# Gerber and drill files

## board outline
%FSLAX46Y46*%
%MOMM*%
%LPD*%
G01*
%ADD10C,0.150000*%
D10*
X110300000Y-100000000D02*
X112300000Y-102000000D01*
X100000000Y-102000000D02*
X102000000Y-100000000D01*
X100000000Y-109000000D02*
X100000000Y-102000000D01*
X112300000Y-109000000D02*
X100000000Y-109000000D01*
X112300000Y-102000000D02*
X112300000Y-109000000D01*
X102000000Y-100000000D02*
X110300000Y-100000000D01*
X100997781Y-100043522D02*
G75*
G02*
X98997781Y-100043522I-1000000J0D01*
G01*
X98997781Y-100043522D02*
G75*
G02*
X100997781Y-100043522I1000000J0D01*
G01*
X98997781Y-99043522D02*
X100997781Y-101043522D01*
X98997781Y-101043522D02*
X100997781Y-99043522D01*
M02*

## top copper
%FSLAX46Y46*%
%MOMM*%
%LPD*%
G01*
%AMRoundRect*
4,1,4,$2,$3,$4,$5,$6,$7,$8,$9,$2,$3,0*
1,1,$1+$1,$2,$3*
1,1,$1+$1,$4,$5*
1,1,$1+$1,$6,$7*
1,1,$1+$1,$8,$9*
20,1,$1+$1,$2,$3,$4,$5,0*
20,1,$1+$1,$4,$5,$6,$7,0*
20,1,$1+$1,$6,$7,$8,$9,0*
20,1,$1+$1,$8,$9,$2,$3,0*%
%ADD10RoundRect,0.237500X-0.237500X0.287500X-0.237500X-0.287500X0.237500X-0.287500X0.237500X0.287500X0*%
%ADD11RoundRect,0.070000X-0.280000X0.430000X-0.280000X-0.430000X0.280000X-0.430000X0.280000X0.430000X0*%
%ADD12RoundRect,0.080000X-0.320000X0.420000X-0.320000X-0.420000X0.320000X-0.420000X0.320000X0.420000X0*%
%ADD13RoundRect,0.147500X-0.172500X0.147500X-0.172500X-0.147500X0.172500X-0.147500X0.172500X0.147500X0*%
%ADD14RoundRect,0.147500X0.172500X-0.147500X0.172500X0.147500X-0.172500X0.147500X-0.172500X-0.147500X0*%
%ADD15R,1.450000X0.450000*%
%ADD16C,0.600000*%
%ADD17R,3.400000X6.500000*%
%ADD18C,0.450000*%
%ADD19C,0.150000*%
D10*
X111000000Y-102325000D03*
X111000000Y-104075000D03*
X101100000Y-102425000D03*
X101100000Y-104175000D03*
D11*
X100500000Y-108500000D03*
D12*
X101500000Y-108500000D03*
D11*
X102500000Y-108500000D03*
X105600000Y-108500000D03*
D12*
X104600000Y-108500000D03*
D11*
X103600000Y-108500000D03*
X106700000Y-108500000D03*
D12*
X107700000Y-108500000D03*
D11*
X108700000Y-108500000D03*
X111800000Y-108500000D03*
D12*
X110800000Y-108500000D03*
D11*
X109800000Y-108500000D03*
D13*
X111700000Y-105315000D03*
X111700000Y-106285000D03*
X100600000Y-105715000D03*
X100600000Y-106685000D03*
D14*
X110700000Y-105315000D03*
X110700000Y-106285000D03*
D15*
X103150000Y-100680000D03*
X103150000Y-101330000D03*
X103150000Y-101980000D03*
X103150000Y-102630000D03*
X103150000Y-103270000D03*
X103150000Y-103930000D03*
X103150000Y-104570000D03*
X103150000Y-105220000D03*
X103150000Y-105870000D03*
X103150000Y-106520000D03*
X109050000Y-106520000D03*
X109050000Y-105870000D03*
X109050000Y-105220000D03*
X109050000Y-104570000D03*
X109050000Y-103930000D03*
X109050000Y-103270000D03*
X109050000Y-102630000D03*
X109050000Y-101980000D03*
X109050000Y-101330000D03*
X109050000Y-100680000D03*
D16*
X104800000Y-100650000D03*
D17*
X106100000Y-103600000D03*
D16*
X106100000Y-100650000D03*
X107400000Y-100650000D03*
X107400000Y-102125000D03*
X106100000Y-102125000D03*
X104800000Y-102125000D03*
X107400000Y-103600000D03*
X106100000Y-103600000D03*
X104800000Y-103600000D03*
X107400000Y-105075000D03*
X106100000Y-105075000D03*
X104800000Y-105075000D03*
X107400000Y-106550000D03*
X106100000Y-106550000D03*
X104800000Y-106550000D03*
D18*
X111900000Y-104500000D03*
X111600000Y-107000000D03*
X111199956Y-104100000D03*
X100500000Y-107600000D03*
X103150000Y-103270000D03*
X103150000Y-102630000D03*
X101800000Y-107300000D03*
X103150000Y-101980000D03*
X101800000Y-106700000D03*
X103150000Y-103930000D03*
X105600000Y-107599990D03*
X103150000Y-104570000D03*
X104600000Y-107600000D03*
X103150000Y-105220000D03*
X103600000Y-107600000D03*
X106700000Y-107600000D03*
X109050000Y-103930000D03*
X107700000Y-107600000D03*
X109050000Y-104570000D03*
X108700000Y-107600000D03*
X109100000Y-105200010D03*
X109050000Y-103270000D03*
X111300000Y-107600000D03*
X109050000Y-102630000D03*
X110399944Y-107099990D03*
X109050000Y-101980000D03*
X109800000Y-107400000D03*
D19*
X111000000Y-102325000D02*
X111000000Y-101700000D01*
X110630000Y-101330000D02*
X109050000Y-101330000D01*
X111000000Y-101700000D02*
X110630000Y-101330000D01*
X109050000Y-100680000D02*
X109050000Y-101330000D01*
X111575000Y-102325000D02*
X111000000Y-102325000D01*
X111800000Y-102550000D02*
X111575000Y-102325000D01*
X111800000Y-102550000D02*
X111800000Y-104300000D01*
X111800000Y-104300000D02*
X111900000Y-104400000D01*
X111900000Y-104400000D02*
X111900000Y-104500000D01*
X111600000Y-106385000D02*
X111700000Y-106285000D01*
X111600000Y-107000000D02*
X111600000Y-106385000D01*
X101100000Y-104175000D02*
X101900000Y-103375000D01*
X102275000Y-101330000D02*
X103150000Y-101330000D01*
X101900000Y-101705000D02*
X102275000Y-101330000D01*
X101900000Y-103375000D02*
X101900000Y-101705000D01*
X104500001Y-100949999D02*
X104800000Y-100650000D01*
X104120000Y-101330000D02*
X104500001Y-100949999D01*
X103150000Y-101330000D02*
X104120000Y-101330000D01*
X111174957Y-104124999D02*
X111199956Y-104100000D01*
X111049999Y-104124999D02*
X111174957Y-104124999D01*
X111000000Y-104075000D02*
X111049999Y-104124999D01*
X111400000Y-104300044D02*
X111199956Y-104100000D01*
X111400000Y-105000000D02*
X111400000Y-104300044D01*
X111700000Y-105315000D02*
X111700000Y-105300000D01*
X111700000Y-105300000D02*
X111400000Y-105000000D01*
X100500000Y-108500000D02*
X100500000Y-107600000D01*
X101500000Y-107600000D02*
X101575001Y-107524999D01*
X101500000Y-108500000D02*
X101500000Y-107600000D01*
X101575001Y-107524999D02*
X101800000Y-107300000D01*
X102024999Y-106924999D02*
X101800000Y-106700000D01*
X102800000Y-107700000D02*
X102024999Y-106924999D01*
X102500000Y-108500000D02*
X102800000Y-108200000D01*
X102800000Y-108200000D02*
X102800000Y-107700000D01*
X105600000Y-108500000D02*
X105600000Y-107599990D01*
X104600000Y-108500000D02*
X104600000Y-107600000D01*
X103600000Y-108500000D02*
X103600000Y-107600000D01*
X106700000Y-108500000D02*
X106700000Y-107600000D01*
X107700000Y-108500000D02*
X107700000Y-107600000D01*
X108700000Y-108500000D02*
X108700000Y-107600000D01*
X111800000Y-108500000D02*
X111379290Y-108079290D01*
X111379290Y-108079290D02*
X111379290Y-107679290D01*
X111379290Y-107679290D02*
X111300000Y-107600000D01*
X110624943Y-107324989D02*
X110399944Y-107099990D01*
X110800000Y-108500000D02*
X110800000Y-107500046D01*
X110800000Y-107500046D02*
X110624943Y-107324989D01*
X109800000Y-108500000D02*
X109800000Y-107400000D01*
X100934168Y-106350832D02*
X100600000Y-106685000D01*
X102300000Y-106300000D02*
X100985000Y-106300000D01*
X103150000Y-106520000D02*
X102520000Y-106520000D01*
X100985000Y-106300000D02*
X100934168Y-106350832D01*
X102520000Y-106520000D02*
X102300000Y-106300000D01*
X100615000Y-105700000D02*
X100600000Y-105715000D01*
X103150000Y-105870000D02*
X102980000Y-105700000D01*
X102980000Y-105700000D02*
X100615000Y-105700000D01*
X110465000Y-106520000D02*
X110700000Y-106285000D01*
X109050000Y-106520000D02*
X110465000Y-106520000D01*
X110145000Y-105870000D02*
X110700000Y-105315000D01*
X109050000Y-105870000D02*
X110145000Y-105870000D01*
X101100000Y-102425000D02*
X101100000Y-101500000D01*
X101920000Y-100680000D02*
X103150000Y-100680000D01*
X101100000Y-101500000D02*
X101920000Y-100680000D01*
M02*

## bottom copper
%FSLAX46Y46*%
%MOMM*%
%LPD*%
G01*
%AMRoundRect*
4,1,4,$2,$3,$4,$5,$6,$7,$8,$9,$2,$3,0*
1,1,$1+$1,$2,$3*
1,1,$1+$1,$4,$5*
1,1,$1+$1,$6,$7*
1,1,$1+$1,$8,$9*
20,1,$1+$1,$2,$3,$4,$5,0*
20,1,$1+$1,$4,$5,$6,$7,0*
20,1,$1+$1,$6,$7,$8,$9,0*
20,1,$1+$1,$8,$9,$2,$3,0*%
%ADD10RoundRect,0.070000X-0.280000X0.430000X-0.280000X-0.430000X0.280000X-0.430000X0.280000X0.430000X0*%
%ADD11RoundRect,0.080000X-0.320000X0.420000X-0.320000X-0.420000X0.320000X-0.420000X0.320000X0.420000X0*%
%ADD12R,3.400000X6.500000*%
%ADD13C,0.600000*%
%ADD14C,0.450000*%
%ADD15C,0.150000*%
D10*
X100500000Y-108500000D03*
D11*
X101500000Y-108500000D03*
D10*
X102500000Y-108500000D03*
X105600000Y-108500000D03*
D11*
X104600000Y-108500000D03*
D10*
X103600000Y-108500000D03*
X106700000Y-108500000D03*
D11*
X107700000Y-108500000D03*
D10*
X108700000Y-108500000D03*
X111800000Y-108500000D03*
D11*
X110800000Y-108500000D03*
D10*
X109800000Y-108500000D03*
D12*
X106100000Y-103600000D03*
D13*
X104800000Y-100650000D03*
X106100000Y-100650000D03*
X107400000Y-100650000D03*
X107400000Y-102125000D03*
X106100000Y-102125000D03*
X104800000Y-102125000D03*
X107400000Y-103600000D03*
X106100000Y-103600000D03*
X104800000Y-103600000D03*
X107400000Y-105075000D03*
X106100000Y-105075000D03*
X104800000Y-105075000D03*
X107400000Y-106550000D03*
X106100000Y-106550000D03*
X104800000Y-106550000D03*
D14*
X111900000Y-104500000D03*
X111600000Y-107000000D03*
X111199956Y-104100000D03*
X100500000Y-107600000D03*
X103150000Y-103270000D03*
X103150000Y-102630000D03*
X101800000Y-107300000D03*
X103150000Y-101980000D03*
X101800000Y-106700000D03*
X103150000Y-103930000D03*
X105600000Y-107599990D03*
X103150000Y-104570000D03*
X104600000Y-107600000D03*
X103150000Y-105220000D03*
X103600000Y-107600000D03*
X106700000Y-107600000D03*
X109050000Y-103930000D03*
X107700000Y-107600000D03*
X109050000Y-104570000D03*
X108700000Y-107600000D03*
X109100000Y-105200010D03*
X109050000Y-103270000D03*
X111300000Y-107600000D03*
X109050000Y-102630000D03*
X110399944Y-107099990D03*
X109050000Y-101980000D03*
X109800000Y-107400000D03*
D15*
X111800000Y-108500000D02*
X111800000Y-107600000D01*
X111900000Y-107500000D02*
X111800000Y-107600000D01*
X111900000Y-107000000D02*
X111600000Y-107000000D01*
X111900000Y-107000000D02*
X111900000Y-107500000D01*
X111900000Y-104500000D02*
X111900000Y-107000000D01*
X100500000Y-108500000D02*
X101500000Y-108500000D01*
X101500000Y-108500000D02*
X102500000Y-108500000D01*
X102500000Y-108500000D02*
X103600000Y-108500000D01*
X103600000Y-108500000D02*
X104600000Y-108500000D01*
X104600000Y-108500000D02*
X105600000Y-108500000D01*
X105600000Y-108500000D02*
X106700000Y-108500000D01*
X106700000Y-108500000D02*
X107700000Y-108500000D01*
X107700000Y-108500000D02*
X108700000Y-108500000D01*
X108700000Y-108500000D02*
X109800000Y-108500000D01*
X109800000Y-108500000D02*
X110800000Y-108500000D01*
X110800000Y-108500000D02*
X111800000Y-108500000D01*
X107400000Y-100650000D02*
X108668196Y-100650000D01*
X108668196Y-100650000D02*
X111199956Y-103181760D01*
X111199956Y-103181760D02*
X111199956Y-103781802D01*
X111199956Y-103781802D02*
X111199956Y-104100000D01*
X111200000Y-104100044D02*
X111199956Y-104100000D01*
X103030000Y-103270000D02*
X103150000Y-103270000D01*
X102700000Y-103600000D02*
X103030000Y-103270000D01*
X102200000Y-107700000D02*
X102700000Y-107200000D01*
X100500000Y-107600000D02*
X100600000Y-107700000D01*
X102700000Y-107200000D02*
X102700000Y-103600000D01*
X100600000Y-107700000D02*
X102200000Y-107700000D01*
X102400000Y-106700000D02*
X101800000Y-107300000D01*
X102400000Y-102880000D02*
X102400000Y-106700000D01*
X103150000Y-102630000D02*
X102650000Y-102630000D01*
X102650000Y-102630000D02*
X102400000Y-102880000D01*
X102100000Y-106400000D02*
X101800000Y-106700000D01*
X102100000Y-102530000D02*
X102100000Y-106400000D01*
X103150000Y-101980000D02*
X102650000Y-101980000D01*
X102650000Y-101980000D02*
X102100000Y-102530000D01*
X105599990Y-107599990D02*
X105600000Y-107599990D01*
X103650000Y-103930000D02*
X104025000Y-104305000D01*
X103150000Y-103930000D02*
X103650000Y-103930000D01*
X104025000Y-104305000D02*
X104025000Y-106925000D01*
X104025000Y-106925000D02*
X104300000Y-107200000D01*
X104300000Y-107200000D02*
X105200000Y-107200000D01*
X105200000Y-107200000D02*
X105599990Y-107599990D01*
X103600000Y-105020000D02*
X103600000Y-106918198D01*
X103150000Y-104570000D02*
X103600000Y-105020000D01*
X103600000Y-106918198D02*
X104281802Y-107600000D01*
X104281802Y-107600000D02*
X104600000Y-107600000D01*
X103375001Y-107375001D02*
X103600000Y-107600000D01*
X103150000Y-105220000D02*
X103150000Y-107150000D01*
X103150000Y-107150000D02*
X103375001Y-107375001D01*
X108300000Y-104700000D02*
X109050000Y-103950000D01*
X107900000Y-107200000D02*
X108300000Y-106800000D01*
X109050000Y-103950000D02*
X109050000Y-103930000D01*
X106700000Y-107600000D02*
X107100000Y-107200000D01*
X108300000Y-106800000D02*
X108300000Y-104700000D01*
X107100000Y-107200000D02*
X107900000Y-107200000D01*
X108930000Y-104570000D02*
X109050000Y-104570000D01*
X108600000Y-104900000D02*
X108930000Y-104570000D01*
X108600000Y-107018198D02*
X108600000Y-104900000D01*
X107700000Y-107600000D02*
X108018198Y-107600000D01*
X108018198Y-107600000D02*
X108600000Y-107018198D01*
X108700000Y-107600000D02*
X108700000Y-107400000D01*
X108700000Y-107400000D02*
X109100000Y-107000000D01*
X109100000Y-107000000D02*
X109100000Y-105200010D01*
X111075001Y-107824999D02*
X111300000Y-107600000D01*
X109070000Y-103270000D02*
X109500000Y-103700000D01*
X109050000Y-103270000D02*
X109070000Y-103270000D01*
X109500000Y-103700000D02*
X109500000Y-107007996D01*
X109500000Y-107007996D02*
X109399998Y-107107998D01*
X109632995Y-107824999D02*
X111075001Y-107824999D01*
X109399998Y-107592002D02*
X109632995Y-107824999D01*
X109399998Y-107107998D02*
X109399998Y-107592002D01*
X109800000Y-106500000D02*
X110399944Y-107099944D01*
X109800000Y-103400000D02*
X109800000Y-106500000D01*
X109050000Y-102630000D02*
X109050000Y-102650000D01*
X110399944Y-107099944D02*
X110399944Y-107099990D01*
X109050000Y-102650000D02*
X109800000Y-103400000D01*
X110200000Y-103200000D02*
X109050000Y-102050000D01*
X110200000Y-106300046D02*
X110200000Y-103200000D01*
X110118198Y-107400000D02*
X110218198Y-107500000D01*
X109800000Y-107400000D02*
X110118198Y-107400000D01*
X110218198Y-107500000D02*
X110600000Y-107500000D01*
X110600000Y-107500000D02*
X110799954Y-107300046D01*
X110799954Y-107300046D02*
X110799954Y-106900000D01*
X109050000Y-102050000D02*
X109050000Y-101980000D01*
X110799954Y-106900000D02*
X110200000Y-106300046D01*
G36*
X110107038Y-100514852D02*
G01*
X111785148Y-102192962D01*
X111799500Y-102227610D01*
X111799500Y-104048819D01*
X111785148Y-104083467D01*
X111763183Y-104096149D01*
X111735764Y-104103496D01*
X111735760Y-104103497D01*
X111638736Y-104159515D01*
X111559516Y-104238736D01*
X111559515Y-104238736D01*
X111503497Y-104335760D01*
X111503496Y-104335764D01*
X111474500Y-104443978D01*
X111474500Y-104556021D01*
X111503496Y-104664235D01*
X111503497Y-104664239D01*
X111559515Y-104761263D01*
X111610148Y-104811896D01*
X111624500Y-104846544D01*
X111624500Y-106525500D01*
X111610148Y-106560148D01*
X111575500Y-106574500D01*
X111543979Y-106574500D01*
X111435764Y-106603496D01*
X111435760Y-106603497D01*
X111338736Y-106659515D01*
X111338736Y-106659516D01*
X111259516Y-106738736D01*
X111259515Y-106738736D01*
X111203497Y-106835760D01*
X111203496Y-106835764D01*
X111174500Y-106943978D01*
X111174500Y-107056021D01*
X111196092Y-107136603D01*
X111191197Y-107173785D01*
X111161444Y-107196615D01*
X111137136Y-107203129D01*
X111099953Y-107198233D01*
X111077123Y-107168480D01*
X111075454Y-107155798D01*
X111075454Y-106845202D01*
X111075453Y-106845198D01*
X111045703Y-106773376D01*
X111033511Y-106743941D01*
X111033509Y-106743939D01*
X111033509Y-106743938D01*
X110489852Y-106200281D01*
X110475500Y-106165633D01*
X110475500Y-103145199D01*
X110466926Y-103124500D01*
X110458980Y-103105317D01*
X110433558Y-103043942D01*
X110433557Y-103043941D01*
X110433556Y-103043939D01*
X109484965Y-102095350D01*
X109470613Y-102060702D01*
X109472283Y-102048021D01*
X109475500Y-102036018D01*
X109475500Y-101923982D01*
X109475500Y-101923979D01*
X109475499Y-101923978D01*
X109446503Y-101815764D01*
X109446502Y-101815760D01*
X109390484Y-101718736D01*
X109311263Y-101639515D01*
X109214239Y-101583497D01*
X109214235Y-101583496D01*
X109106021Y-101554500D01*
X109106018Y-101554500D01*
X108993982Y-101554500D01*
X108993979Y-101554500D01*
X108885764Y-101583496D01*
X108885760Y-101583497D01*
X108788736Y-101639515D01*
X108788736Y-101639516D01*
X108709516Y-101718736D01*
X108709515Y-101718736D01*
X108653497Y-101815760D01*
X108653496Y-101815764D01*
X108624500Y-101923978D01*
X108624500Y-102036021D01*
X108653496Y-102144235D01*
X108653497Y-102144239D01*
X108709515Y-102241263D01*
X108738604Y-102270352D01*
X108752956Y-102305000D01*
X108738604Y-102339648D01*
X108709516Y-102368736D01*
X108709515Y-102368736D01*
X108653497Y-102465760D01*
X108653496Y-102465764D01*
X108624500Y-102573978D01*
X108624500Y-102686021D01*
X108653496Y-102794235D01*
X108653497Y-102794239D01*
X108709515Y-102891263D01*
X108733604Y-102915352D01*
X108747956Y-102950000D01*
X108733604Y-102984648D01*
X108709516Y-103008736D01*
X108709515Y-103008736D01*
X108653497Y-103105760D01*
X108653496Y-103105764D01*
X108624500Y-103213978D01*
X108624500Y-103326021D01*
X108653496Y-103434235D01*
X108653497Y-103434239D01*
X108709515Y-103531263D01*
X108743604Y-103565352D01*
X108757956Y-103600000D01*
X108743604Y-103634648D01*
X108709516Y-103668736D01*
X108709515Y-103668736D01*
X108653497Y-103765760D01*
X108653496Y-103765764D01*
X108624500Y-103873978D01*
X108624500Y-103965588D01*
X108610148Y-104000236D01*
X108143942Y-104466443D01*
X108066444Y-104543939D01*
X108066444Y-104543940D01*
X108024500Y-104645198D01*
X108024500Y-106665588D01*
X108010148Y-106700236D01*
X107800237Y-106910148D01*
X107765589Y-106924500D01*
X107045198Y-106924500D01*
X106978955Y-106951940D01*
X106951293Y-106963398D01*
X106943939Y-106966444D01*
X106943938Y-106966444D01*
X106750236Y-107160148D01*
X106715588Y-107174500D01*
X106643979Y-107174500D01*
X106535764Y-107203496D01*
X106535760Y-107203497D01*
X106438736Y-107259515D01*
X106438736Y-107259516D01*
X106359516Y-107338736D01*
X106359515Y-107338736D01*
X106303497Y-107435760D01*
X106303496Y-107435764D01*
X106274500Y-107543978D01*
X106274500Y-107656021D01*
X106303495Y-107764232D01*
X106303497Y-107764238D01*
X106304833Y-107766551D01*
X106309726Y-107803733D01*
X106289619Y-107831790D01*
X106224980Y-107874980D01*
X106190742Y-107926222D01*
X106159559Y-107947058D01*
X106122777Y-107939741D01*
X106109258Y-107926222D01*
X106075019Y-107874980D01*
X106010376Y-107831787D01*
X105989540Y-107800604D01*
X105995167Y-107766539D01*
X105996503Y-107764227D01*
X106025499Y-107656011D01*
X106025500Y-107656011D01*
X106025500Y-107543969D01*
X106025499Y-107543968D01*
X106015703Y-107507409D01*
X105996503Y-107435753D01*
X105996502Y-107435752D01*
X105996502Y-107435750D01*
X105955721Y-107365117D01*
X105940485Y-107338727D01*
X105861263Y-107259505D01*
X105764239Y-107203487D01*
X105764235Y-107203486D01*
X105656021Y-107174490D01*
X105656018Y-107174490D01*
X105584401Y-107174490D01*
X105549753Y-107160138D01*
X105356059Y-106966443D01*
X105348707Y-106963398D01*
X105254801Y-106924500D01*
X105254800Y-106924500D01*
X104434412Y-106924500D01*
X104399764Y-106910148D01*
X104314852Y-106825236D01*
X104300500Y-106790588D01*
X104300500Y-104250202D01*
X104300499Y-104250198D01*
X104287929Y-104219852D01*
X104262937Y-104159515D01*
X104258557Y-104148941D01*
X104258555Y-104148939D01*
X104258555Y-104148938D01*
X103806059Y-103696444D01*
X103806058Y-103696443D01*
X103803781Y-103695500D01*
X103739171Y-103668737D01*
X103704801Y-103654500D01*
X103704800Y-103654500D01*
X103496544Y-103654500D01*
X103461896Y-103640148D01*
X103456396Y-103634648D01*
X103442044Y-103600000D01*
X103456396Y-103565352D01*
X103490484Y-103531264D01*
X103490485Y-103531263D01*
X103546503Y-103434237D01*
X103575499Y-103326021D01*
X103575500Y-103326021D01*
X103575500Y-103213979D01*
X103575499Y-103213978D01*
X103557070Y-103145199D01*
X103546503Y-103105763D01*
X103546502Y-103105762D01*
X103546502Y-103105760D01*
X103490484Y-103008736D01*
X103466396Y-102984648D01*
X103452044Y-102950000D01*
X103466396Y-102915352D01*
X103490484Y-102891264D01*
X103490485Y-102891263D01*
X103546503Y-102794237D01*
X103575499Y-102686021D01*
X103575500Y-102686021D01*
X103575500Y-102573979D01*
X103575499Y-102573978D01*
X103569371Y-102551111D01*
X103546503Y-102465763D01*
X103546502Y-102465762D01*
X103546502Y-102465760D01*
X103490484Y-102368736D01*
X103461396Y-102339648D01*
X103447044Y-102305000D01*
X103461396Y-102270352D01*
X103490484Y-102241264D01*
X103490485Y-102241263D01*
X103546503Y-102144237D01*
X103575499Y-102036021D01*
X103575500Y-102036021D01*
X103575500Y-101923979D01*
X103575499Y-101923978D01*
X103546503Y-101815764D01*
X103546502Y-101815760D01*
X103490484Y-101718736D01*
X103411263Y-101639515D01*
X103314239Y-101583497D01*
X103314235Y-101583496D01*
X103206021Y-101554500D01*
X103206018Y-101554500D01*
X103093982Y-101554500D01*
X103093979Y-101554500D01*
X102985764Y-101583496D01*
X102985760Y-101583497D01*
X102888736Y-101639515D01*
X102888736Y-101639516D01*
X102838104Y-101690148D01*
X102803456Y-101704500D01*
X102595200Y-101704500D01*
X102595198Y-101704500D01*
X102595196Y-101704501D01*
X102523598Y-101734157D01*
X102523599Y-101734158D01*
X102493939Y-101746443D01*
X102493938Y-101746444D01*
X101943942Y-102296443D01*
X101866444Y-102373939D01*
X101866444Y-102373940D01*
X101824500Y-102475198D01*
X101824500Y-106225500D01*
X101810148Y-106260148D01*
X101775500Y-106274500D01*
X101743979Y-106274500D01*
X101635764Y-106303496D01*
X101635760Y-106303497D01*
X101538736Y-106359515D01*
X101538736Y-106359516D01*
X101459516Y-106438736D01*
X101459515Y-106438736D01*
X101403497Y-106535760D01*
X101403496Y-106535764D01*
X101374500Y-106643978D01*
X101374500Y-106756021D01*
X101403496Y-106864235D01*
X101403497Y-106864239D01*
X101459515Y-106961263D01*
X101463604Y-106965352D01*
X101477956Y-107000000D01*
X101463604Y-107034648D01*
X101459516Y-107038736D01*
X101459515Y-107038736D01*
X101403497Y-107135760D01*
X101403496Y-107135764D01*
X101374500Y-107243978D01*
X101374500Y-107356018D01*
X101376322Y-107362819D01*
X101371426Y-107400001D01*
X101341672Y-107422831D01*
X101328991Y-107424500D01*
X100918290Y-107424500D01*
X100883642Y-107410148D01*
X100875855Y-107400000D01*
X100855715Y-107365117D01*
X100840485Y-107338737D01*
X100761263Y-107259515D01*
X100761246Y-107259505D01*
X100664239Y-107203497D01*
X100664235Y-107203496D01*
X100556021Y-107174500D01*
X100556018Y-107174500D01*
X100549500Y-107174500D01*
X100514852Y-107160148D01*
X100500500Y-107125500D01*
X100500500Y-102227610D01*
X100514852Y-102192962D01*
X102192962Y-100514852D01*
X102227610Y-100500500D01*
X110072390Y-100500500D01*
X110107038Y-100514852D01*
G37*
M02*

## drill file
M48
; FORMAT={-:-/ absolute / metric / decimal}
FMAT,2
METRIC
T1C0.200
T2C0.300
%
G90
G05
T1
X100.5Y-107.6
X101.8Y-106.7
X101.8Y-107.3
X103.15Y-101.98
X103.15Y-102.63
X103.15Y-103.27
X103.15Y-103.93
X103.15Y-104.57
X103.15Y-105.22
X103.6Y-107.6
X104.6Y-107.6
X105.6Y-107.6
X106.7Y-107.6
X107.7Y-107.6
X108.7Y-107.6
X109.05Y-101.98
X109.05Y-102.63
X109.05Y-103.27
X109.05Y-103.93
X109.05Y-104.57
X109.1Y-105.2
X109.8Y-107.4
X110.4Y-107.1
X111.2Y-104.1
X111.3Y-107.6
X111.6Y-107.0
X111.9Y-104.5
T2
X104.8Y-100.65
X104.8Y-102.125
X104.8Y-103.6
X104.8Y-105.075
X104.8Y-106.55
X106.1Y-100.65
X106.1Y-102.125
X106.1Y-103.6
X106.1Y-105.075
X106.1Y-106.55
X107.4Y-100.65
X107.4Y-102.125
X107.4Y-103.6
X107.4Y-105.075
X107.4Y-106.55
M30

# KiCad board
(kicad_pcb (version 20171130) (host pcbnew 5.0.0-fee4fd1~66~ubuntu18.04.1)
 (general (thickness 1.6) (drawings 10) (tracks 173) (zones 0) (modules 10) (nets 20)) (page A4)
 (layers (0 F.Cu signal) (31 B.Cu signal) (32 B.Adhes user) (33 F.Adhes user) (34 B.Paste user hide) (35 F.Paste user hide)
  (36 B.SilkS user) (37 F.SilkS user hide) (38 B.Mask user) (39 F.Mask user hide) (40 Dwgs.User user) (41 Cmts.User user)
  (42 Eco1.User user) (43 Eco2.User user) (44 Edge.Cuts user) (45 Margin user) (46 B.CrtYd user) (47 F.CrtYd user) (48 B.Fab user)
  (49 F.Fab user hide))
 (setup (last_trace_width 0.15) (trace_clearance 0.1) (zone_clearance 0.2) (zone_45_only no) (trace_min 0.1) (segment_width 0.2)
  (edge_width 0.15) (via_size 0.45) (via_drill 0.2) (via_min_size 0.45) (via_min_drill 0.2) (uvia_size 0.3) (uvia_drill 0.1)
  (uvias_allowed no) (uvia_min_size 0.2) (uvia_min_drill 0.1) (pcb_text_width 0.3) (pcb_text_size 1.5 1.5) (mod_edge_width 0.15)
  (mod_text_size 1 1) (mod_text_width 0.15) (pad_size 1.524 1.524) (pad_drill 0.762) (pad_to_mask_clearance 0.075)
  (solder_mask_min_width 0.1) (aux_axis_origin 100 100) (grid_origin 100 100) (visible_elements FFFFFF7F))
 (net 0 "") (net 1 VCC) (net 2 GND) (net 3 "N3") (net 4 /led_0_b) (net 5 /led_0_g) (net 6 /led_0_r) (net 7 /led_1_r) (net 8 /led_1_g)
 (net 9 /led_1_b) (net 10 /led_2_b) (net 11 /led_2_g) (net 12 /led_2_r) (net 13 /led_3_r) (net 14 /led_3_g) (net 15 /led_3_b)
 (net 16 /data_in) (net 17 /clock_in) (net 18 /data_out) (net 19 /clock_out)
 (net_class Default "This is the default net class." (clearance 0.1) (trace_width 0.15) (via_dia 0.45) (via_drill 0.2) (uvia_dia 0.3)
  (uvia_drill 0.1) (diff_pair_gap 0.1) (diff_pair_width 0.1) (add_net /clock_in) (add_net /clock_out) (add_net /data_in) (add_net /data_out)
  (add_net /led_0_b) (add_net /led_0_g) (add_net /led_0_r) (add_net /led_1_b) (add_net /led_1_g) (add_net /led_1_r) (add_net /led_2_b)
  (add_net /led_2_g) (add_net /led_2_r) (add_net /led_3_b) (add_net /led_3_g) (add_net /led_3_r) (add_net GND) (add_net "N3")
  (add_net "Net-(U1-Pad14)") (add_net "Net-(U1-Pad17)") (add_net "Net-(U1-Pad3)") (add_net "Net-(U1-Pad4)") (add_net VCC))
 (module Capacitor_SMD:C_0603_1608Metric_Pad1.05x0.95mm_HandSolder (layer F.Cu) (at 111 103.2 270)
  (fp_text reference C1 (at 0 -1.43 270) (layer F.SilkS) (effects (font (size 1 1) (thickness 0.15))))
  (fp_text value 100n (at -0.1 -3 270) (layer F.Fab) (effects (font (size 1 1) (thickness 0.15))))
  (pad 1 smd roundrect (at -0.875 0 270) (size 1.05 0.95) (layers F.Cu F.Paste F.Mask) (roundrect_rratio 0.25) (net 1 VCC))
  (pad 2 smd roundrect (at 0.875 0 270) (size 1.05 0.95) (layers F.Cu F.Paste F.Mask) (roundrect_rratio 0.25) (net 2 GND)))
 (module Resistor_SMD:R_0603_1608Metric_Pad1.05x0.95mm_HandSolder (layer F.Cu) (at 101.1 103.3 270)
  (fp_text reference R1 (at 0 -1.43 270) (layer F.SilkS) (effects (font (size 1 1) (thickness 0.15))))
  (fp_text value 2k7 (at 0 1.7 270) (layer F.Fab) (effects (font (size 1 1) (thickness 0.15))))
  (pad 1 smd roundrect (at -0.875 0 270) (size 1.05 0.95) (layers F.Cu F.Paste F.Mask) (roundrect_rratio 0.25) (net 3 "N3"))
  (pad 2 smd roundrect (at 0.875 0 270) (size 1.05 0.95) (layers F.Cu F.Paste F.Mask) (roundrect_rratio 0.25) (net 2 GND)))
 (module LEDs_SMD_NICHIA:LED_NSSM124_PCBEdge (layer F.Cu) (at 101.5 109 270)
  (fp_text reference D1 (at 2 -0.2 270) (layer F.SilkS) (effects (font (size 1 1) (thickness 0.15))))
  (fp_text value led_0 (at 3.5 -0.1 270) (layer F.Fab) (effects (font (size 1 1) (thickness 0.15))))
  (pad 3 smd roundrect (at -0.5 1 270) (size 1 0.7) (layers F.Cu F.Mask) (roundrect_rratio 0.1) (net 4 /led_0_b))
  (pad 2 smd roundrect (at -0.5 0 270) (size 1 0.8) (layers F.Cu F.Mask) (roundrect_rratio 0.1) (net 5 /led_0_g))
  (pad 4 smd roundrect (at -0.5 1 270) (size 1 0.7) (layers B.Cu B.Mask) (roundrect_rratio 0.1) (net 1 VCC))
  (pad 5 smd roundrect (at -0.5 0 270) (size 1 0.8) (layers B.Cu B.Mask) (roundrect_rratio 0.1) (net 1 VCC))
  (pad 6 smd roundrect (at -0.5 -1 270) (size 1 0.7) (layers B.Cu B.Mask) (roundrect_rratio 0.1) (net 1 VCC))
  (pad 1 smd roundrect (at -0.5 -1 270) (size 1 0.7) (layers F.Cu F.Mask) (roundrect_rratio 0.1) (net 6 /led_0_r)))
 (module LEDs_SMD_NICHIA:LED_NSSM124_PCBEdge (layer F.Cu) (at 104.6 109 270)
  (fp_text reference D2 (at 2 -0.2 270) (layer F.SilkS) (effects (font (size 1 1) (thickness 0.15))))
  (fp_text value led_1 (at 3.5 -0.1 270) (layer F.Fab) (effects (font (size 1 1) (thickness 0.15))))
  (pad 1 smd roundrect (at -0.5 -1 270) (size 1 0.7) (layers F.Cu F.Mask) (roundrect_rratio 0.1) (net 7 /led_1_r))
  (pad 6 smd roundrect (at -0.5 -1 270) (size 1 0.7) (layers B.Cu B.Mask) (roundrect_rratio 0.1) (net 1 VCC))
  (pad 5 smd roundrect (at -0.5 0 270) (size 1 0.8) (layers B.Cu B.Mask) (roundrect_rratio 0.1) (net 1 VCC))
  (pad 4 smd roundrect (at -0.5 1 270) (size 1 0.7) (layers B.Cu B.Mask) (roundrect_rratio 0.1) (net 1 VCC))
  (pad 2 smd roundrect (at -0.5 0 270) (size 1 0.8) (layers F.Cu F.Mask) (roundrect_rratio 0.1) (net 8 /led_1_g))
  (pad 3 smd roundrect (at -0.5 1 270) (size 1 0.7) (layers F.Cu F.Mask) (roundrect_rratio 0.1) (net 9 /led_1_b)))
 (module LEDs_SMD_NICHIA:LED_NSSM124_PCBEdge (layer F.Cu) (at 107.7 109 270)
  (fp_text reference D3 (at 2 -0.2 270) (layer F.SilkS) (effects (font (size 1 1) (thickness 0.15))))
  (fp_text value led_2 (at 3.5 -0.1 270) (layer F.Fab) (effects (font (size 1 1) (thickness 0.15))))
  (pad 3 smd roundrect (at -0.5 1 270) (size 1 0.7) (layers F.Cu F.Mask) (roundrect_rratio 0.1) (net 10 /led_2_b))
  (pad 2 smd roundrect (at -0.5 0 270) (size 1 0.8) (layers F.Cu F.Mask) (roundrect_rratio 0.1) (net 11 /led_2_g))
  (pad 4 smd roundrect (at -0.5 1 270) (size 1 0.7) (layers B.Cu B.Mask) (roundrect_rratio 0.1) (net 1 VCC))
  (pad 5 smd roundrect (at -0.5 0 270) (size 1 0.8) (layers B.Cu B.Mask) (roundrect_rratio 0.1) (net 1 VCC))
  (pad 6 smd roundrect (at -0.5 -1 270) (size 1 0.7) (layers B.Cu B.Mask) (roundrect_rratio 0.1) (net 1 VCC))
  (pad 1 smd roundrect (at -0.5 -1 270) (size 1 0.7) (layers F.Cu F.Mask) (roundrect_rratio 0.1) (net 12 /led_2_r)))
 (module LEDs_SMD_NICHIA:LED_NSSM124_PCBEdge (layer F.Cu) (at 110.8 109 270)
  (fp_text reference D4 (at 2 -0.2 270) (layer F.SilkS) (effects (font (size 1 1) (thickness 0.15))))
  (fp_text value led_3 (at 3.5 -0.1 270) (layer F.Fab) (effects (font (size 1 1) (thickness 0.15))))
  (pad 1 smd roundrect (at -0.5 -1 270) (size 1 0.7) (layers F.Cu F.Mask) (roundrect_rratio 0.1) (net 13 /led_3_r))
  (pad 6 smd roundrect (at -0.5 -1 270) (size 1 0.7) (layers B.Cu B.Mask) (roundrect_rratio 0.1) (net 1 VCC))
  (pad 5 smd roundrect (at -0.5 0 270) (size 1 0.8) (layers B.Cu B.Mask) (roundrect_rratio 0.1) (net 1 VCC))
  (pad 4 smd roundrect (at -0.5 1 270) (size 1 0.7) (layers B.Cu B.Mask) (roundrect_rratio 0.1) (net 1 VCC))
  (pad 2 smd roundrect (at -0.5 0 270) (size 1 0.8) (layers F.Cu F.Mask) (roundrect_rratio 0.1) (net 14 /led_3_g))
  (pad 3 smd roundrect (at -0.5 1 270) (size 1 0.7) (layers F.Cu F.Mask) (roundrect_rratio 0.1) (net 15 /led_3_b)))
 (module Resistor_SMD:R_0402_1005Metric (layer F.Cu) (at 111.7 105.8 270)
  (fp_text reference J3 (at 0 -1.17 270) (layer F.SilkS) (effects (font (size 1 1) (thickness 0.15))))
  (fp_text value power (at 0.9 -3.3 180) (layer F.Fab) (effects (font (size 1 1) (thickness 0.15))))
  (pad 1 smd roundrect (at -0.485 0 270) (size 0.59 0.64) (layers F.Cu F.Paste F.Mask) (roundrect_rratio 0.25) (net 2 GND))
  (pad 2 smd roundrect (at 0.485 0 270) (size 0.59 0.64) (layers F.Cu F.Paste F.Mask) (roundrect_rratio 0.25) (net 1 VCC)))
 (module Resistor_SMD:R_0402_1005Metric (layer F.Cu) (at 100.6 106.2 270)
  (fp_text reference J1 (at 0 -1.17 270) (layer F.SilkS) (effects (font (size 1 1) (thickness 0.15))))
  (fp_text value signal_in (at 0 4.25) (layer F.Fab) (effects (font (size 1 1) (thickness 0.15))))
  (pad 1 smd roundrect (at -0.485 0 270) (size 0.59 0.64) (layers F.Cu F.Paste F.Mask) (roundrect_rratio 0.25) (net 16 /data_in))
  (pad 2 smd roundrect (at 0.485 0 270) (size 0.59 0.64) (layers F.Cu F.Paste F.Mask) (roundrect_rratio 0.25) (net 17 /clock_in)))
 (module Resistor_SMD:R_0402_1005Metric (layer F.Cu) (at 110.7 105.8 90)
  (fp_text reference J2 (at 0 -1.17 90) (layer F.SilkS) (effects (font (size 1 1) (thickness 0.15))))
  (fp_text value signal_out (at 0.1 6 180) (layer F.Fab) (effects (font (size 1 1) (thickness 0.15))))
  (pad 2 smd roundrect (at 0.485 0 90) (size 0.59 0.64) (layers F.Cu F.Paste F.Mask) (roundrect_rratio 0.25) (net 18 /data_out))
  (pad 1 smd roundrect (at -0.485 0 90) (size 0.59 0.64) (layers F.Cu F.Paste F.Mask) (roundrect_rratio 0.25) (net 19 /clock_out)))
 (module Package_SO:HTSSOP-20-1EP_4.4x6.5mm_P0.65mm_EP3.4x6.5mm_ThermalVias (layer F.Cu) (at 106.1 103.6)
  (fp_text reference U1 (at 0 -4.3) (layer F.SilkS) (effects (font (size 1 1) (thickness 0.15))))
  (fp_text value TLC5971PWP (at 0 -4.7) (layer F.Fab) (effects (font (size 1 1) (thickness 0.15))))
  (pad 21 smd rect (at 0 0) (size 3.4 6.5) (layers B.Cu) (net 2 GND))
  (pad 1 smd rect (at -2.95 -2.92) (size 1.45 0.45) (layers F.Cu F.Paste F.Mask) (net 3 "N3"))
  (pad 2 smd rect (at -2.95 -2.27) (size 1.45 0.45) (layers F.Cu F.Paste F.Mask) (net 2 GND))
  (pad 3 smd rect (at -2.95 -1.62) (size 1.45 0.45) (layers F.Cu F.Paste F.Mask) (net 6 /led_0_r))
  (pad 4 smd rect (at -2.95 -0.97) (size 1.45 0.45) (layers F.Cu F.Paste F.Mask) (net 5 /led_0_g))
  (pad 5 smd rect (at -2.95 -0.33) (size 1.45 0.45) (layers F.Cu F.Paste F.Mask) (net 4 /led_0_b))
  (pad 6 smd rect (at -2.95 0.33) (size 1.45 0.45) (layers F.Cu F.Paste F.Mask) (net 7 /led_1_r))
  (pad 7 smd rect (at -2.95 0.97) (size 1.45 0.45) (layers F.Cu F.Paste F.Mask) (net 8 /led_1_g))
  (pad 8 smd rect (at -2.95 1.62) (size 1.45 0.45) (layers F.Cu F.Paste F.Mask) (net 9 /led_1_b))
  (pad 9 smd rect (at -2.95 2.27) (size 1.45 0.45) (layers F.Cu F.Paste F.Mask) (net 16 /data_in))
  (pad 10 smd rect (at -2.95 2.92) (size 1.45 0.45) (layers F.Cu F.Paste F.Mask) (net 17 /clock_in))
  (pad 11 smd rect (at 2.95 2.92) (size 1.45 0.45) (layers F.Cu F.Paste F.Mask) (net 19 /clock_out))
  (pad 12 smd rect (at 2.95 2.27) (size 1.45 0.45) (layers F.Cu F.Paste F.Mask) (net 18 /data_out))
  (pad 13 smd rect (at 2.95 1.62) (size 1.45 0.45) (layers F.Cu F.Paste F.Mask) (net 12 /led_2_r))
  (pad 14 smd rect (at 2.95 0.97) (size 1.45 0.45) (layers F.Cu F.Paste F.Mask) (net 11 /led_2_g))
  (pad 15 smd rect (at 2.95 0.33) (size 1.45 0.45) (layers F.Cu F.Paste F.Mask) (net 10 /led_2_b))
  (pad 16 smd rect (at 2.95 -0.33) (size 1.45 0.45) (layers F.Cu F.Paste F.Mask) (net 13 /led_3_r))
  (pad 17 smd rect (at 2.95 -0.97) (size 1.45 0.45) (layers F.Cu F.Paste F.Mask) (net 14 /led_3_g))
  (pad 18 smd rect (at 2.95 -1.62) (size 1.45 0.45) (layers F.Cu F.Paste F.Mask) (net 15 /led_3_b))
  (pad 19 smd rect (at 2.95 -2.27) (size 1.45 0.45) (layers F.Cu F.Paste F.Mask) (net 1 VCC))
  (pad 20 smd rect (at 2.95 -2.92) (size 1.45 0.45) (layers F.Cu F.Paste F.Mask) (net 1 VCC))
  (pad 21 thru_hole circle (at -1.3 -2.95) (size 0.6 0.6) (drill 0.3) (layers *.Cu) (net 2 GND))
  (pad 21 smd rect (at 0 0) (size 3.4 6.5) (layers F.Cu F.Mask) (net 2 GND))
  (pad "" smd rect (at -0.85 -2.2125) (size 1.4 1.075) (layers F.Paste))
  (pad "" smd rect (at 0.85 -2.2125) (size 1.4 1.075) (layers F.Paste))
  (pad "" smd rect (at 0.85 -0.7375) (size 1.4 1.075) (layers F.Paste))
  (pad "" smd rect (at -0.85 -0.7375) (size 1.4 1.075) (layers F.Paste))
  (pad "" smd rect (at 0.85 0.7375) (size 1.4 1.075) (layers F.Paste))
  (pad "" smd rect (at -0.85 0.7375) (size 1.4 1.075) (layers F.Paste))
  (pad "" smd rect (at 0.85 2.2125) (size 1.4 1.075) (layers F.Paste))
  (pad "" smd rect (at -0.85 2.2125) (size 1.4 1.075) (layers F.Paste))
  (pad 21 thru_hole circle (at 0 -2.95) (size 0.6 0.6) (drill 0.3) (layers *.Cu) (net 2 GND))
  (pad 21 thru_hole circle (at 1.3 -2.95) (size 0.6 0.6) (drill 0.3) (layers *.Cu) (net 2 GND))
  (pad 21 thru_hole circle (at 1.3 -1.475) (size 0.6 0.6) (drill 0.3) (layers *.Cu) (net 2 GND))
  (pad 21 thru_hole circle (at 0 -1.475) (size 0.6 0.6) (drill 0.3) (layers *.Cu) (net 2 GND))
  (pad 21 thru_hole circle (at -1.3 -1.475) (size 0.6 0.6) (drill 0.3) (layers *.Cu) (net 2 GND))
  (pad 21 thru_hole circle (at 1.3 0) (size 0.6 0.6) (drill 0.3) (layers *.Cu) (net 2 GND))
  (pad 21 thru_hole circle (at 0 0) (size 0.6 0.6) (drill 0.3) (layers *.Cu) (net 2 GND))
  (pad 21 thru_hole circle (at -1.3 0) (size 0.6 0.6) (drill 0.3) (layers *.Cu) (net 2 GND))
  (pad 21 thru_hole circle (at 1.3 1.475) (size 0.6 0.6) (drill 0.3) (layers *.Cu) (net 2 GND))
  (pad 21 thru_hole circle (at 0 1.475) (size 0.6 0.6) (drill 0.3) (layers *.Cu) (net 2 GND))
  (pad 21 thru_hole circle (at -1.3 1.475) (size 0.6 0.6) (drill 0.3) (layers *.Cu) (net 2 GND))
  (pad 21 thru_hole circle (at 1.3 2.95) (size 0.6 0.6) (drill 0.3) (layers *.Cu) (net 2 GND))
  (pad 21 thru_hole circle (at 0 2.95) (size 0.6 0.6) (drill 0.3) (layers *.Cu) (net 2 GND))
  (pad 21 thru_hole circle (at -1.3 2.95) (size 0.6 0.6) (drill 0.3) (layers *.Cu) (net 2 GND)))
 (gr_line (start 110.3 100) (end 112.3 102) (layer Edge.Cuts) (width 0.15))
 (gr_line (start 100 102) (end 102 100) (layer Edge.Cuts) (width 0.15))
 (gr_line (start 100 109) (end 100 102) (layer Edge.Cuts) (width 0.15))
 (gr_line (start 112.3 109) (end 100 109) (layer Edge.Cuts) (width 0.15))
 (gr_line (start 112.3 102) (end 112.3 109) (layer Edge.Cuts) (width 0.15))
 (gr_line (start 102 100) (end 110.3 100) (layer Edge.Cuts) (width 0.15))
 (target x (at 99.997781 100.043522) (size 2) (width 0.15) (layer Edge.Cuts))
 (segment (start 111 102.325) (end 111 101.7) (width 0.15) (layer F.Cu) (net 1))
 (segment (start 110.63 101.33) (end 109.05 101.33) (width 0.15) (layer F.Cu) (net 1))
 (segment (start 111 101.7) (end 110.63 101.33) (width 0.15) (layer F.Cu) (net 1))
 (segment (start 109.05 100.68) (end 109.05 101.33) (width 0.15) (layer F.Cu) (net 1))
 (segment (start 111.575 102.325) (end 111 102.325) (width 0.15) (layer F.Cu) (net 1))
 (segment (start 111.8 102.55) (end 111.575 102.325) (width 0.15) (layer F.Cu) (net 1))
 (segment (start 111.8 108.5) (end 111.8 107.6) (width 0.15) (layer B.Cu) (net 1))
 (segment (start 111.8 102.55) (end 111.8 104.3) (width 0.15) (layer F.Cu) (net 1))
 (via (at 111.9 104.5) (size 0.45) (drill 0.2) (layers F.Cu B.Cu) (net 1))
 (segment (start 111.8 104.3) (end 111.9 104.4) (width 0.15) (layer F.Cu) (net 1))
 (segment (start 111.9 104.4) (end 111.9 104.5) (width 0.15) (layer F.Cu) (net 1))
 (segment (start 111.9 107.5) (end 111.8 107.6) (width 0.15) (layer B.Cu) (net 1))
 (segment (start 111.9 107) (end 111.6 107) (width 0.15) (layer B.Cu) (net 1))
 (segment (start 111.9 107) (end 111.9 107.5) (width 0.15) (layer B.Cu) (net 1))
 (via (at 111.6 107) (size 0.45) (drill 0.2) (layers F.Cu B.Cu) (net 1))
 (segment (start 111.9 104.5) (end 111.9 107) (width 0.15) (layer B.Cu) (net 1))
 (segment (start 111.6 106.385) (end 111.7 106.285) (width 0.15) (layer F.Cu) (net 1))
 (segment (start 111.6 107) (end 111.6 106.385) (width 0.15) (layer F.Cu) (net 1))
 (segment (start 100.5 108.5) (end 101.5 108.5) (width 0.15) (layer B.Cu) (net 1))
 (segment (start 101.5 108.5) (end 102.5 108.5) (width 0.15) (layer B.Cu) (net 1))
 (segment (start 102.5 108.5) (end 103.6 108.5) (width 0.15) (layer B.Cu) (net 1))
 (segment (start 103.6 108.5) (end 104.6 108.5) (width 0.15) (layer B.Cu) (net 1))
 (segment (start 104.6 108.5) (end 105.6 108.5) (width 0.15) (layer B.Cu) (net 1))
 (segment (start 105.6 108.5) (end 106.7 108.5) (width 0.15) (layer B.Cu) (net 1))
 (segment (start 106.7 108.5) (end 107.7 108.5) (width 0.15) (layer B.Cu) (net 1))
 (segment (start 107.7 108.5) (end 108.7 108.5) (width 0.15) (layer B.Cu) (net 1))
 (segment (start 108.7 108.5) (end 109.8 108.5) (width 0.15) (layer B.Cu) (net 1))
 (segment (start 109.8 108.5) (end 110.8 108.5) (width 0.15) (layer B.Cu) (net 1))
 (segment (start 110.8 108.5) (end 111.8 108.5) (width 0.15) (layer B.Cu) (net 1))
 (segment (start 101.1 104.175) (end 101.9 103.375) (width 0.15) (layer F.Cu) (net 2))
 (segment (start 102.275 101.33) (end 103.15 101.33) (width 0.15) (layer F.Cu) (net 2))
 (segment (start 101.9 101.705) (end 102.275 101.33) (width 0.15) (layer F.Cu) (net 2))
 (segment (start 101.9 103.375) (end 101.9 101.705) (width 0.15) (layer F.Cu) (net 2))
 (segment (start 104.500001 100.949999) (end 104.8 100.65) (width 0.15) (layer F.Cu) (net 2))
 (segment (start 104.12 101.33) (end 104.500001 100.949999) (width 0.15) (layer F.Cu) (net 2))
 (segment (start 103.15 101.33) (end 104.12 101.33) (width 0.15) (layer F.Cu) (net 2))
 (segment (start 107.4 100.65) (end 108.668196 100.65) (width 0.15) (layer B.Cu) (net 2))
 (segment (start 108.668196 100.65) (end 111.199956 103.18176) (width 0.15) (layer B.Cu) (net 2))
 (segment (start 111.174957 104.124999) (end 111.199956 104.1) (width 0.15) (layer F.Cu) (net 2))
 (via (at 111.199956 104.1) (size 0.45) (drill 0.2) (layers F.Cu B.Cu) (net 2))
 (segment (start 111.049999 104.124999) (end 111.174957 104.124999) (width 0.15) (layer F.Cu) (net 2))
 (segment (start 111.199956 103.18176) (end 111.199956 103.781802) (width 0.15) (layer B.Cu) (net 2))
 (segment (start 111 104.075) (end 111.049999 104.124999) (width 0.15) (layer F.Cu) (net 2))
 (segment (start 111.199956 103.781802) (end 111.199956 104.1) (width 0.15) (layer B.Cu) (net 2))
 (segment (start 111.2 104.100044) (end 111.199956 104.1) (width 0.15) (layer B.Cu) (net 2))
 (segment (start 111.4 104.300044) (end 111.199956 104.1) (width 0.15) (layer F.Cu) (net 2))
 (segment (start 111.4 105) (end 111.4 104.300044) (width 0.15) (layer F.Cu) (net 2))
 (segment (start 111.7 105.315) (end 111.7 105.3) (width 0.15) (layer F.Cu) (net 2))
 (segment (start 111.7 105.3) (end 111.4 105) (width 0.15) (layer F.Cu) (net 2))
 (via (at 100.5 107.6) (size 0.45) (drill 0.2) (layers F.Cu B.Cu) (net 4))
 (segment (start 100.5 108.5) (end 100.5 107.6) (width 0.15) (layer F.Cu) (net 4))
 (via (at 103.15 103.27) (size 0.45) (drill 0.2) (layers F.Cu B.Cu) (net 4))
 (segment (start 103.03 103.27) (end 103.15 103.27) (width 0.15) (layer B.Cu) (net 4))
 (segment (start 102.7 103.6) (end 103.03 103.27) (width 0.15) (layer B.Cu) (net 4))
 (segment (start 102.2 107.7) (end 102.7 107.2) (width 0.15) (layer B.Cu) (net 4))
 (segment (start 100.5 107.6) (end 100.6 107.7) (width 0.15) (layer B.Cu) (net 4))
 (segment (start 102.7 107.2) (end 102.7 103.6) (width 0.15) (layer B.Cu) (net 4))
 (segment (start 100.6 107.7) (end 102.2 107.7) (width 0.15) (layer B.Cu) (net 4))
 (via (at 103.15 102.63) (size 0.45) (drill 0.2) (layers F.Cu B.Cu) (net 5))
 (via (at 101.8 107.3) (size 0.45) (drill 0.2) (layers F.Cu B.Cu) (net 5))
 (segment (start 101.5 107.6) (end 101.575001 107.524999) (width 0.15) (layer F.Cu) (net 5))
 (segment (start 101.5 108.5) (end 101.5 107.6) (width 0.15) (layer F.Cu) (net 5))
 (segment (start 101.575001 107.524999) (end 101.8 107.3) (width 0.15) (layer F.Cu) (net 5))
 (segment (start 102.4 106.7) (end 101.8 107.3) (width 0.15) (layer B.Cu) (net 5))
 (segment (start 102.4 102.88) (end 102.4 106.7) (width 0.15) (layer B.Cu) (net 5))
 (segment (start 103.15 102.63) (end 102.65 102.63) (width 0.15) (layer B.Cu) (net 5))
 (segment (start 102.65 102.63) (end 102.4 102.88) (width 0.15) (layer B.Cu) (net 5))
 (via (at 103.15 101.98) (size 0.45) (drill 0.2) (layers F.Cu B.Cu) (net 6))
 (via (at 101.8 106.7) (size 0.45) (drill 0.2) (layers F.Cu B.Cu) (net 6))
 (segment (start 102.1 106.4) (end 101.8 106.7) (width 0.15) (layer B.Cu) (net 6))
 (segment (start 102.1 102.53) (end 102.1 106.4) (width 0.15) (layer B.Cu) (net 6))
 (segment (start 103.15 101.98) (end 102.65 101.98) (width 0.15) (layer B.Cu) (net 6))
 (segment (start 102.65 101.98) (end 102.1 102.53) (width 0.15) (layer B.Cu) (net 6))
 (segment (start 102.024999 106.924999) (end 101.8 106.7) (width 0.15) (layer F.Cu) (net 6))
 (segment (start 102.8 107.7) (end 102.024999 106.924999) (width 0.15) (layer F.Cu) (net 6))
 (segment (start 102.5 108.5) (end 102.8 108.2) (width 0.15) (layer F.Cu) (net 6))
 (segment (start 102.8 108.2) (end 102.8 107.7) (width 0.15) (layer F.Cu) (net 6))
 (via (at 103.15 103.93) (size 0.45) (drill 0.2) (layers F.Cu B.Cu) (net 7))
 (segment (start 105.6 108.5) (end 105.6 107.59999) (width 0.15) (layer F.Cu) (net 7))
 (via (at 105.6 107.59999) (size 0.45) (drill 0.2) (layers F.Cu B.Cu) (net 7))
 (segment (start 105.59999 107.59999) (end 105.6 107.59999) (width 0.15) (layer B.Cu) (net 7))
 (segment (start 103.65 103.93) (end 104.025 104.305) (width 0.15) (layer B.Cu) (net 7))
 (segment (start 103.15 103.93) (end 103.65 103.93) (width 0.15) (layer B.Cu) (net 7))
 (segment (start 104.025 104.305) (end 104.025 106.925) (width 0.15) (layer B.Cu) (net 7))
 (segment (start 104.025 106.925) (end 104.3 107.2) (width 0.15) (layer B.Cu) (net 7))
 (segment (start 104.3 107.2) (end 105.2 107.2) (width 0.15) (layer B.Cu) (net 7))
 (segment (start 105.2 107.2) (end 105.59999 107.59999) (width 0.15) (layer B.Cu) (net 7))
 (via (at 103.15 104.57) (size 0.45) (drill 0.2) (layers F.Cu B.Cu) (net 8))
 (segment (start 104.6 108.5) (end 104.6 107.6) (width 0.15) (layer F.Cu) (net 8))
 (via (at 104.6 107.6) (size 0.45) (drill 0.2) (layers F.Cu B.Cu) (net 8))
 (segment (start 103.6 105.02) (end 103.6 106.918198) (width 0.15) (layer B.Cu) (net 8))
 (segment (start 103.15 104.57) (end 103.6 105.02) (width 0.15) (layer B.Cu) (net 8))
 (segment (start 103.6 106.918198) (end 104.281802 107.6) (width 0.15) (layer B.Cu) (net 8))
 (segment (start 104.281802 107.6) (end 104.6 107.6) (width 0.15) (layer B.Cu) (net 8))
 (via (at 103.15 105.22) (size 0.45) (drill 0.2) (layers F.Cu B.Cu) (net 9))
 (segment (start 103.6 108.5) (end 103.6 107.6) (width 0.15) (layer F.Cu) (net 9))
 (segment (start 103.375001 107.375001) (end 103.6 107.6) (width 0.15) (layer B.Cu) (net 9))
 (via (at 103.6 107.6) (size 0.45) (drill 0.2) (layers F.Cu B.Cu) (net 9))
 (segment (start 103.15 105.22) (end 103.15 107.15) (width 0.15) (layer B.Cu) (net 9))
 (segment (start 103.15 107.15) (end 103.375001 107.375001) (width 0.15) (layer B.Cu) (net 9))
 (via (at 106.7 107.6) (size 0.45) (drill 0.2) (layers F.Cu B.Cu) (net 10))
 (segment (start 106.7 108.5) (end 106.7 107.6) (width 0.15) (layer F.Cu) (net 10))
 (via (at 109.05 103.93) (size 0.45) (drill 0.2) (layers F.Cu B.Cu) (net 10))
 (segment (start 108.3 104.7) (end 109.05 103.95) (width 0.15) (layer B.Cu) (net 10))
 (segment (start 107.9 107.2) (end 108.3 106.8) (width 0.15) (layer B.Cu) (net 10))
 (segment (start 109.05 103.95) (end 109.05 103.93) (width 0.15) (layer B.Cu) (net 10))
 (segment (start 106.7 107.6) (end 107.1 107.2) (width 0.15) (layer B.Cu) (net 10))
 (segment (start 108.3 106.8) (end 108.3 104.7) (width 0.15) (layer B.Cu) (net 10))
 (segment (start 107.1 107.2) (end 107.9 107.2) (width 0.15) (layer B.Cu) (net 10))
 (via (at 107.7 107.6) (size 0.45) (drill 0.2) (layers F.Cu B.Cu) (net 11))
 (segment (start 107.7 108.5) (end 107.7 107.6) (width 0.15) (layer F.Cu) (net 11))
 (via (at 109.05 104.57) (size 0.45) (drill 0.2) (layers F.Cu B.Cu) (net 11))
 (segment (start 108.93 104.57) (end 109.05 104.57) (width 0.15) (layer B.Cu) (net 11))
 (segment (start 108.6 104.9) (end 108.93 104.57) (width 0.15) (layer B.Cu) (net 11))
 (segment (start 108.6 107.018198) (end 108.6 104.9) (width 0.15) (layer B.Cu) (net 11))
 (segment (start 107.7 107.6) (end 108.018198 107.6) (width 0.15) (layer B.Cu) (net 11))
 (segment (start 108.018198 107.6) (end 108.6 107.018198) (width 0.15) (layer B.Cu) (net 11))
 (via (at 108.7 107.6) (size 0.45) (drill 0.2) (layers F.Cu B.Cu) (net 12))
 (segment (start 108.7 108.5) (end 108.7 107.6) (width 0.15) (layer F.Cu) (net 12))
 (via (at 109.1 105.20001) (size 0.45) (drill 0.2) (layers F.Cu B.Cu) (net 12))
 (segment (start 108.7 107.6) (end 108.7 107.4) (width 0.15) (layer B.Cu) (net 12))
 (segment (start 108.7 107.4) (end 109.1 107) (width 0.15) (layer B.Cu) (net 12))
 (segment (start 109.1 107) (end 109.1 105.20001) (width 0.15) (layer B.Cu) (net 12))
 (via (at 109.05 103.27) (size 0.45) (drill 0.2) (layers F.Cu B.Cu) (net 13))
 (via (at 111.3 107.6) (size 0.45) (drill 0.2) (layers F.Cu B.Cu) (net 13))
 (segment (start 111.8 108.5) (end 111.37929 108.07929) (width 0.15) (layer F.Cu) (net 13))
 (segment (start 111.37929 108.07929) (end 111.37929 107.67929) (width 0.15) (layer F.Cu) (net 13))
 (segment (start 111.37929 107.67929) (end 111.3 107.6) (width 0.15) (layer F.Cu) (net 13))
 (segment (start 111.075001 107.824999) (end 111.3 107.6) (width 0.15) (layer B.Cu) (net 13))
 (segment (start 109.07 103.27) (end 109.5 103.7) (width 0.15) (layer B.Cu) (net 13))
 (segment (start 109.05 103.27) (end 109.07 103.27) (width 0.15) (layer B.Cu) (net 13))
 (segment (start 109.5 103.7) (end 109.5 107.007996) (width 0.15) (layer B.Cu) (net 13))
 (segment (start 109.5 107.007996) (end 109.399998 107.107998) (width 0.15) (layer B.Cu) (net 13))
 (segment (start 109.632995 107.824999) (end 111.075001 107.824999) (width 0.15) (layer B.Cu) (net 13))
 (segment (start 109.399998 107.592002) (end 109.632995 107.824999) (width 0.15) (layer B.Cu) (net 13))
 (segment (start 109.399998 107.107998) (end 109.399998 107.592002) (width 0.15) (layer B.Cu) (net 13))
 (via (at 109.05 102.63) (size 0.45) (drill 0.2) (layers F.Cu B.Cu) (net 14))
 (via (at 110.399944 107.09999) (size 0.45) (drill 0.2) (layers F.Cu B.Cu) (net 14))
 (segment (start 110.624943 107.324989) (end 110.399944 107.09999) (width 0.15) (layer F.Cu) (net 14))
 (segment (start 110.8 108.5) (end 110.8 107.500046) (width 0.15) (layer F.Cu) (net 14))
 (segment (start 110.8 107.500046) (end 110.624943 107.324989) (width 0.15) (layer F.Cu) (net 14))
 (segment (start 109.8 106.5) (end 110.399944 107.099944) (width 0.15) (layer B.Cu) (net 14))
 (segment (start 109.8 103.4) (end 109.8 106.5) (width 0.15) (layer B.Cu) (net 14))
 (segment (start 109.05 102.63) (end 109.05 102.65) (width 0.15) (layer B.Cu) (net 14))
 (segment (start 110.399944 107.099944) (end 110.399944 107.09999) (width 0.15) (layer B.Cu) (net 14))
 (segment (start 109.05 102.65) (end 109.8 103.4) (width 0.15) (layer B.Cu) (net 14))
 (via (at 109.05 101.98) (size 0.45) (drill 0.2) (layers F.Cu B.Cu) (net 15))
 (via (at 109.8 107.4) (size 0.45) (drill 0.2) (layers F.Cu B.Cu) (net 15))
 (segment (start 109.8 108.5) (end 109.8 107.4) (width 0.15) (layer F.Cu) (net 15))
 (segment (start 110.2 103.2) (end 109.05 102.05) (width 0.15) (layer B.Cu) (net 15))
 (segment (start 110.2 106.300046) (end 110.2 103.2) (width 0.15) (layer B.Cu) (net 15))
 (segment (start 110.118198 107.4) (end 110.218198 107.5) (width 0.15) (layer B.Cu) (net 15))
 (segment (start 109.8 107.4) (end 110.118198 107.4) (width 0.15) (layer B.Cu) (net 15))
 (segment (start 110.218198 107.5) (end 110.6 107.5) (width 0.15) (layer B.Cu) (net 15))
 (segment (start 110.6 107.5) (end 110.799954 107.300046) (width 0.15) (layer B.Cu) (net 15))
 (segment (start 110.799954 107.300046) (end 110.799954 106.9) (width 0.15) (layer B.Cu) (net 15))
 (segment (start 109.05 102.05) (end 109.05 101.98) (width 0.15) (layer B.Cu) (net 15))
 (segment (start 110.799954 106.9) (end 110.2 106.300046) (width 0.15) (layer B.Cu) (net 15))
 (segment (start 100.934168 106.350832) (end 100.6 106.685) (width 0.15) (layer F.Cu) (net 17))
 (segment (start 102.3 106.3) (end 100.985 106.3) (width 0.15) (layer F.Cu) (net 17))
 (segment (start 103.15 106.52) (end 102.52 106.52) (width 0.15) (layer F.Cu) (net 17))
 (segment (start 100.985 106.3) (end 100.934168 106.350832) (width 0.15) (layer F.Cu) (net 17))
 (segment (start 102.52 106.52) (end 102.3 106.3) (width 0.15) (layer F.Cu) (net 17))
 (segment (start 100.615 105.7) (end 100.6 105.715) (width 0.15) (layer F.Cu) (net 16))
 (segment (start 103.15 105.87) (end 102.98 105.7) (width 0.15) (layer F.Cu) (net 16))
 (segment (start 102.98 105.7) (end 100.615 105.7) (width 0.15) (layer F.Cu) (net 16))
 (segment (start 110.465 106.52) (end 110.7 106.285) (width 0.15) (layer F.Cu) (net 19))
 (segment (start 109.05 106.52) (end 110.465 106.52) (width 0.15) (layer F.Cu) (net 19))
 (segment (start 110.145 105.87) (end 110.7 105.315) (width 0.15) (layer F.Cu) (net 18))
 (segment (start 109.05 105.87) (end 110.145 105.87) (width 0.15) (layer F.Cu) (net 18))
 (segment (start 101.1 102.425) (end 101.1 101.5) (width 0.15) (layer F.Cu) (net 3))
 (segment (start 101.92 100.68) (end 103.15 100.68) (width 0.15) (layer F.Cu) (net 3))
 (segment (start 101.1 101.5) (end 101.92 100.68) (width 0.15) (layer F.Cu) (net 3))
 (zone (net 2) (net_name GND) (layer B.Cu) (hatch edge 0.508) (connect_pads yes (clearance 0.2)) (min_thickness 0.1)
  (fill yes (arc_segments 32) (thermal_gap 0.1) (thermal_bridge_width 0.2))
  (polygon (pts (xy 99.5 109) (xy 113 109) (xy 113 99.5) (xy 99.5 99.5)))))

